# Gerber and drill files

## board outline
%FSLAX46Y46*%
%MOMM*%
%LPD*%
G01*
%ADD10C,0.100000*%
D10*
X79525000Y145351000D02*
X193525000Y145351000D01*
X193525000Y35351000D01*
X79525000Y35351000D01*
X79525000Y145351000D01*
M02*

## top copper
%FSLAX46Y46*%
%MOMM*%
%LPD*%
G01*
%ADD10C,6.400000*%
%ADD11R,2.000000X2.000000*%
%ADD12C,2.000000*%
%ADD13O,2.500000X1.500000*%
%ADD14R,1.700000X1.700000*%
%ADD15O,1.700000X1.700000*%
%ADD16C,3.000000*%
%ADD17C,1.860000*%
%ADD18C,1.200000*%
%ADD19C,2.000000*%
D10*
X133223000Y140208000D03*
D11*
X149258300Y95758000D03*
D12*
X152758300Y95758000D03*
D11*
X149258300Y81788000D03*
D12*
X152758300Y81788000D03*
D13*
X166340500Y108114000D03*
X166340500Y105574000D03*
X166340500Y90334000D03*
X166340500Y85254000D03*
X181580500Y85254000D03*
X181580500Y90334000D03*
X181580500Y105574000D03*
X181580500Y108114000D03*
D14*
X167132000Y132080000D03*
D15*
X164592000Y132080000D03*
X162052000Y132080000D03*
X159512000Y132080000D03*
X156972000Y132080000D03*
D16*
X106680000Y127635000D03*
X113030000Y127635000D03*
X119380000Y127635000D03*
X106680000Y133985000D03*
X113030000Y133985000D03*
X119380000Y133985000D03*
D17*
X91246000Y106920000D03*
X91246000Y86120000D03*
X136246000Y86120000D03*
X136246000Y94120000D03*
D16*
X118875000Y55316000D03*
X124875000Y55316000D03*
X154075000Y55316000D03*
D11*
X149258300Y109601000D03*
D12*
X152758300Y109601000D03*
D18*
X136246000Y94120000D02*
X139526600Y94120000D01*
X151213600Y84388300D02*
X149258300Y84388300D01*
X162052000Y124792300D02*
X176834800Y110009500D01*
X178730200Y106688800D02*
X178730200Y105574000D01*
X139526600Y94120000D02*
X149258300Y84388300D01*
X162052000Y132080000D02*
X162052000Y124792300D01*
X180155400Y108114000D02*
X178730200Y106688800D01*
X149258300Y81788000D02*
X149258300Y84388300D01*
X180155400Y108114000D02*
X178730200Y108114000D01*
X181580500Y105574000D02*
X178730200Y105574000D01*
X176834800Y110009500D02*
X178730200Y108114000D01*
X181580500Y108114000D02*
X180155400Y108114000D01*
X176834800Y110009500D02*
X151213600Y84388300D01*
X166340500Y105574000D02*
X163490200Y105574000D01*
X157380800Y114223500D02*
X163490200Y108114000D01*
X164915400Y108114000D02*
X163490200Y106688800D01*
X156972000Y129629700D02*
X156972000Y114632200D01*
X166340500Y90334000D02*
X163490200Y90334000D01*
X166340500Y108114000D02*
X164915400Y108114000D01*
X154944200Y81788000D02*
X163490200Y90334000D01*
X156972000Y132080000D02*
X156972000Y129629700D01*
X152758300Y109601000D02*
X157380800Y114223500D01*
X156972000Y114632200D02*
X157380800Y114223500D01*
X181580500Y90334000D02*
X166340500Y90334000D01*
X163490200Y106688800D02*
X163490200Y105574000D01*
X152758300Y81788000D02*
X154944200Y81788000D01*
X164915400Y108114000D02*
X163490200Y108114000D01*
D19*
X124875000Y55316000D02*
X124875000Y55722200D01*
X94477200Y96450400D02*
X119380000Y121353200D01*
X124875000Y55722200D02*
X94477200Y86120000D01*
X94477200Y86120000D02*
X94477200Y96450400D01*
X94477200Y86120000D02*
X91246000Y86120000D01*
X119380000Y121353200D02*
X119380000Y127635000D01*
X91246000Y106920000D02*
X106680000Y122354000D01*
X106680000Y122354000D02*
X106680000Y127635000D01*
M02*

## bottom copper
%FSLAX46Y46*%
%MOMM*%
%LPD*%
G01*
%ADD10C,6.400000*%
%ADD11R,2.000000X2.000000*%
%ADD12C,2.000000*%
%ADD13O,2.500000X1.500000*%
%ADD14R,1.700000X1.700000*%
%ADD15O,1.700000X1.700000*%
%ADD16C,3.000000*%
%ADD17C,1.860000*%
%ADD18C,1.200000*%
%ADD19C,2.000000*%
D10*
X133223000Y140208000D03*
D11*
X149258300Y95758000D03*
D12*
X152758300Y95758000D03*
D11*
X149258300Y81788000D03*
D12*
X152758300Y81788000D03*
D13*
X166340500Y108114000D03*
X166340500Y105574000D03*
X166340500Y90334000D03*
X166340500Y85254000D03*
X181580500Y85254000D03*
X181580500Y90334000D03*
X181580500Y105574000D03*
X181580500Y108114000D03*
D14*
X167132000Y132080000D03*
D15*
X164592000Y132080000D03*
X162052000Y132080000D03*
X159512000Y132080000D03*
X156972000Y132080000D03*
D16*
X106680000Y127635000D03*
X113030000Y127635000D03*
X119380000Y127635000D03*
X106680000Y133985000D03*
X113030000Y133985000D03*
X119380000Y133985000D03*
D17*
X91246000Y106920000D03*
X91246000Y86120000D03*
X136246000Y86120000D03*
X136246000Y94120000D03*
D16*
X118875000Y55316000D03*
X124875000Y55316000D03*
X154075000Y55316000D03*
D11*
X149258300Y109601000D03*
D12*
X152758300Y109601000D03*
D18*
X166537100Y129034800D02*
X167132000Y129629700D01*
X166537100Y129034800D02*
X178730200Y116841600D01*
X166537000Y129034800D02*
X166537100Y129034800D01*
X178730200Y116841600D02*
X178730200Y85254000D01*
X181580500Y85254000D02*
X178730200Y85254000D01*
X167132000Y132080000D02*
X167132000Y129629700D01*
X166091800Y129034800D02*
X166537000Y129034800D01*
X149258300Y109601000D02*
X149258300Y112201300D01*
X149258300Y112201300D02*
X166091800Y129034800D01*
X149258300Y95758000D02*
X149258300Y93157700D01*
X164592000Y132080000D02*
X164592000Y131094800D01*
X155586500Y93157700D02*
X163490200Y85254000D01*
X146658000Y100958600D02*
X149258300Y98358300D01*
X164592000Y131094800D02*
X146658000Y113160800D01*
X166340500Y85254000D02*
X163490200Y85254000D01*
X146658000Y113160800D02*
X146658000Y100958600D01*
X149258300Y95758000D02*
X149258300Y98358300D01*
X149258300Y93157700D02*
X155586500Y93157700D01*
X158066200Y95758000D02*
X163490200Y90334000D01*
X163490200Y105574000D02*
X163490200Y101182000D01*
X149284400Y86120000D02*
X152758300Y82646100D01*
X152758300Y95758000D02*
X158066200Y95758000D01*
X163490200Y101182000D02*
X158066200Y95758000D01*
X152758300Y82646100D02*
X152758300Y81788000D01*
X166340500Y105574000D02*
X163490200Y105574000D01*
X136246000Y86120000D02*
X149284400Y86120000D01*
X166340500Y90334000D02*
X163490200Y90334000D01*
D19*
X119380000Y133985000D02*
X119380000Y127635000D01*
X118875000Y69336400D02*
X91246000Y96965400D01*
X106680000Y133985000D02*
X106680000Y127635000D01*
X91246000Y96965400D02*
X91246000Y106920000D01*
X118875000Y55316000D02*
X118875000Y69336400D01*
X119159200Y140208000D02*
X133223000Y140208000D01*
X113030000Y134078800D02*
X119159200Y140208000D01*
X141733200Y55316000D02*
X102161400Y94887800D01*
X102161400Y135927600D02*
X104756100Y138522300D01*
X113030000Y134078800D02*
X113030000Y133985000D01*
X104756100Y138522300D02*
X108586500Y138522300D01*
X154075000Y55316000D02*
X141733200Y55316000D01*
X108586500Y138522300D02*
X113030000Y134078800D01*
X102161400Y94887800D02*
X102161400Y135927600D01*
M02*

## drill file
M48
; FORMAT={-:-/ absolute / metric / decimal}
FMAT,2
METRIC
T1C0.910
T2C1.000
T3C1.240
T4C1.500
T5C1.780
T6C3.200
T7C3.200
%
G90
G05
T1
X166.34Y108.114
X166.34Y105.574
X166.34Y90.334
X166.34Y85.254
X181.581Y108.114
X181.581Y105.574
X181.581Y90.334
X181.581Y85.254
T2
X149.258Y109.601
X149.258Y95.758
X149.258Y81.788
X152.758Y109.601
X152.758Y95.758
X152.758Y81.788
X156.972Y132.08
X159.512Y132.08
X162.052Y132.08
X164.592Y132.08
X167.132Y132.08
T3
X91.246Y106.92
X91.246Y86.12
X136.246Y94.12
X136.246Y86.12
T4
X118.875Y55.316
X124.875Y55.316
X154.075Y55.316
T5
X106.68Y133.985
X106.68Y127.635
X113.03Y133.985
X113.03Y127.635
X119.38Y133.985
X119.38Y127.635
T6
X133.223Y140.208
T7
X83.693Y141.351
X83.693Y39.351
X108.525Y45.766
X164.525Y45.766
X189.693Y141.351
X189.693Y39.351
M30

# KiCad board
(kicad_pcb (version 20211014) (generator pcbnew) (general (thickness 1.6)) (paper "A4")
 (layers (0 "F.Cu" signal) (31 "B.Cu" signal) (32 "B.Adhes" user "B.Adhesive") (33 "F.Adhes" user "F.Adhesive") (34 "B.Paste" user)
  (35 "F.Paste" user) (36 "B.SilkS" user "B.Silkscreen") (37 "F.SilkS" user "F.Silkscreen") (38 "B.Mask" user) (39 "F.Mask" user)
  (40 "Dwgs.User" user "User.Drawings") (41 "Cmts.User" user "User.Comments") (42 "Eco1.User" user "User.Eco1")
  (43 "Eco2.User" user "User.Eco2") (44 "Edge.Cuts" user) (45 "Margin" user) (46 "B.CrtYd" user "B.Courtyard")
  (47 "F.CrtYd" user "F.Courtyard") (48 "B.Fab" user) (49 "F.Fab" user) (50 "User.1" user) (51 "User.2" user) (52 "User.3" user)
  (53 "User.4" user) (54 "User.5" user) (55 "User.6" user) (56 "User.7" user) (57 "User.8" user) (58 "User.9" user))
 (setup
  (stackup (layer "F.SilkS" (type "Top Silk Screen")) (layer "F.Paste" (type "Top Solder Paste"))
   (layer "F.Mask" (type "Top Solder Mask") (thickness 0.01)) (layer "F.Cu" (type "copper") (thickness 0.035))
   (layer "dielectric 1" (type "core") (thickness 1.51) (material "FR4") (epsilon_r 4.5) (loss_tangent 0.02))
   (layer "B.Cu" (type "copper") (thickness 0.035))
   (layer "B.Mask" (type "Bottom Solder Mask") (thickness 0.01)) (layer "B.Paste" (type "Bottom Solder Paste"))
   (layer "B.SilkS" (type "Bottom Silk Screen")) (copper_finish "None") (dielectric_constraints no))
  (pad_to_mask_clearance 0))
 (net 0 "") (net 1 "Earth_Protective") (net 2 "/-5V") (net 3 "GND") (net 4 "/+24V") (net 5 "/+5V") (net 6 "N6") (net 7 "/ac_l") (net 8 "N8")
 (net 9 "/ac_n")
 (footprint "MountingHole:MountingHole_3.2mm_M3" (layer "F.Cu") (at 189.693 -141.351)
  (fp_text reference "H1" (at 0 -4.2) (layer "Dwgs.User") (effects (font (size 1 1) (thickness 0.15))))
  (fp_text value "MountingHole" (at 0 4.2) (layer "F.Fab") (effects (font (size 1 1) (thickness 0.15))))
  (pad "" np_thru_hole circle (at 0 0) (size 3.2 3.2) (drill 3.2) (layers *.Cu *.Mask)))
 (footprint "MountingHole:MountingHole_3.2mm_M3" (layer "F.Cu") (at 83.693 -39.351)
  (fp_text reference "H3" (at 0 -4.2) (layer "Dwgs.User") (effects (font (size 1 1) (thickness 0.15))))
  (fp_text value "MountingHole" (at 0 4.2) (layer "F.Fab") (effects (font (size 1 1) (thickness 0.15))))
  (pad "" np_thru_hole circle (at 0 0) (size 3.2 3.2) (drill 3.2) (layers *.Cu *.Mask)))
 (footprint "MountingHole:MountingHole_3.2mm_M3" (layer "F.Cu") (at 83.693 -141.351)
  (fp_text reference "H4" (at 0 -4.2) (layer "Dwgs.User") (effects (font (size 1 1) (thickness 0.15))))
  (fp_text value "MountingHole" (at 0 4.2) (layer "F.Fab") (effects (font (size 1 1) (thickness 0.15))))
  (pad "" np_thru_hole circle (at 0 0) (size 3.2 3.2) (drill 3.2) (layers *.Cu *.Mask)))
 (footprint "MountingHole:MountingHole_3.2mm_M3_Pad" (layer "F.Cu") (at 133.223 -140.208)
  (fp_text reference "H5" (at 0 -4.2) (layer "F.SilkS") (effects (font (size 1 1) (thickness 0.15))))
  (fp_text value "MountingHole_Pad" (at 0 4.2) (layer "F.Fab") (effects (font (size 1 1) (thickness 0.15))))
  (pad "1" thru_hole circle (at 0 0) (size 6.4 6.4) (drill 3.2) (layers *.Cu *.Mask) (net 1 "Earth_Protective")))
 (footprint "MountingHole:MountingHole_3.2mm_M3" (layer "F.Cu") (at 189.693 -39.351)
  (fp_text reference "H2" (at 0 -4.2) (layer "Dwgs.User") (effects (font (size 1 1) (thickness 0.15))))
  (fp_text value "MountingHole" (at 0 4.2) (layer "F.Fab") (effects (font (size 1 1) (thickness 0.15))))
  (pad "" np_thru_hole circle (at 0 0) (size 3.2 3.2) (drill 3.2) (layers *.Cu *.Mask)))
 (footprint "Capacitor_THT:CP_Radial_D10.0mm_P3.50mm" (layer "F.Cu") (at 149.2583 -95.758)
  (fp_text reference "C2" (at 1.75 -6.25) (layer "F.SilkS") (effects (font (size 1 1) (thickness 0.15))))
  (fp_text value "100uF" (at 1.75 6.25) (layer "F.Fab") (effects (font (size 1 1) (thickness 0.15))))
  (pad "1" thru_hole rect (at 0 0) (size 2 2) (drill 1) (layers *.Cu *.Mask) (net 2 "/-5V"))
  (pad "2" thru_hole circle (at 3.5 0) (size 2 2) (drill 1) (layers *.Cu *.Mask) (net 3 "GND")))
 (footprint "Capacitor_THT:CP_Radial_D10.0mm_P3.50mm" (layer "F.Cu") (at 149.2583 -81.788)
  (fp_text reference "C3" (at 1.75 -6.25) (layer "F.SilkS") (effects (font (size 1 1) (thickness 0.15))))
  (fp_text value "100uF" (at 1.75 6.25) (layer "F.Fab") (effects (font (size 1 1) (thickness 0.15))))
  (pad "1" thru_hole rect (at 0 0) (size 2 2) (drill 1) (layers *.Cu *.Mask) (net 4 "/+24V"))
  (pad "2" thru_hole circle (at 3.5 0) (size 2 2) (drill 1) (layers *.Cu *.Mask) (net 3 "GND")))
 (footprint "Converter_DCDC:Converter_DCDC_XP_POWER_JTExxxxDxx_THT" (layer "F.Cu") (at 166.3405 -108.114)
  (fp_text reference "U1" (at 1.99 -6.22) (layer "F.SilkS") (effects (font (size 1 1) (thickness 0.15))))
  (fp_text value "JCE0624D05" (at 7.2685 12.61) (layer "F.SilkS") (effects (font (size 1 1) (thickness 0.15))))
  (pad "2" thru_hole oval (at 0 0) (size 2.5 1.5) (drill 0.91) (layers *.Cu *.Mask) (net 3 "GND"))
  (pad "3" thru_hole oval (at 0 2.54) (size 2.5 1.5) (drill 0.91) (layers *.Cu *.Mask) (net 3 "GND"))
  (pad "9" thru_hole oval (at 0 17.78) (size 2.5 1.5) (drill 0.91) (layers *.Cu *.Mask) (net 3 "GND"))
  (pad "11" thru_hole oval (at 0 22.86) (size 2.5 1.5) (drill 0.91) (layers *.Cu *.Mask) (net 2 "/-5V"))
  (pad "14" thru_hole oval (at 15.24 22.86) (size 2.5 1.5) (drill 0.91) (layers *.Cu *.Mask) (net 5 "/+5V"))
  (pad "16" thru_hole oval (at 15.24 17.78) (size 2.5 1.5) (drill 0.91) (layers *.Cu *.Mask) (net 3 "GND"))
  (pad "22" thru_hole oval (at 15.24 2.54) (size 2.5 1.5) (drill 0.91) (layers *.Cu *.Mask) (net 4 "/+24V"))
  (pad "23" thru_hole oval (at 15.24 0) (size 2.5 1.5) (drill 0.91) (layers *.Cu *.Mask) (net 4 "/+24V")))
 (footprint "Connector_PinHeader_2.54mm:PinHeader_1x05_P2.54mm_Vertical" (layer "F.Cu") (at 167.132 -132.08 -90)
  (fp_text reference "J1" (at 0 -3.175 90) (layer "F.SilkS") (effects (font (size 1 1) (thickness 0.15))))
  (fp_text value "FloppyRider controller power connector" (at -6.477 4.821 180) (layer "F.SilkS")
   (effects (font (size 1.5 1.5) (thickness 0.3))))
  (pad "1" thru_hole rect (at 0 0 270) (size 1.7 1.7) (drill 1) (layers *.Cu *.Mask) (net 5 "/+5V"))
  (pad "2" thru_hole oval (at 0 2.54 270) (size 1.7 1.7) (drill 1) (layers *.Cu *.Mask) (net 2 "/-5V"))
  (pad "3" thru_hole oval (at 0 5.08 270) (size 1.7 1.7) (drill 1) (layers *.Cu *.Mask) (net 4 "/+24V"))
  (pad "4" thru_hole oval (at 0 7.62 270) (size 1.7 1.7) (drill 1) (layers *.Cu *.Mask) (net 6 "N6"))
  (pad "5" thru_hole oval (at 0 10.16 270) (size 1.7 1.7) (drill 1) (layers *.Cu *.Mask) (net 3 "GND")))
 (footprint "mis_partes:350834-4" (layer "F.Cu") (at 102.87 -123.825)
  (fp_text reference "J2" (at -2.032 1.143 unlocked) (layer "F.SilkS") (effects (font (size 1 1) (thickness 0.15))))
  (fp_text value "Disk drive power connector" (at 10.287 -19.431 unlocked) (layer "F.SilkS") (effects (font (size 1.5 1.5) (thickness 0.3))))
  (pad "1" thru_hole circle (at 3.81 -3.81) (size 3 3) (drill 1.78) (layers *.Cu *.Mask) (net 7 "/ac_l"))
  (pad "2" thru_hole circle (at 10.16 -3.81) (size 3 3) (drill 1.78) (layers *.Cu *.Mask) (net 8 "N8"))
  (pad "3" thru_hole circle (at 16.51 -3.81) (size 3 3) (drill 1.78) (layers *.Cu *.Mask) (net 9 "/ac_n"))
  (pad "4" thru_hole circle (at 3.81 -10.16) (size 3 3) (drill 1.78) (layers *.Cu *.Mask) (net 7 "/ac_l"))
  (pad "5" thru_hole circle (at 10.16 -10.16) (size 3 3) (drill 1.78) (layers *.Cu *.Mask) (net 1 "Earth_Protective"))
  (pad "6" thru_hole circle (at 16.51 -10.16) (size 3 3) (drill 1.78) (layers *.Cu *.Mask) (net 9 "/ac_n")))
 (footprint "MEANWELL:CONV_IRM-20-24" (layer "F.Cu") (at 114.046 -96.52)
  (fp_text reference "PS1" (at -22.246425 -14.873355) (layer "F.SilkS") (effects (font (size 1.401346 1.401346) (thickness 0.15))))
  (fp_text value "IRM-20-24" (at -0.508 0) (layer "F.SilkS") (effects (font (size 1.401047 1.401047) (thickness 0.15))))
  (pad "1" thru_hole circle locked (at -22.8 -10.4) (size 1.86 1.86) (drill 1.24) (layers *.Cu *.Mask) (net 7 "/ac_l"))
  (pad "2" thru_hole circle locked (at -22.8 10.4) (size 1.86 1.86) (drill 1.24) (layers *.Cu *.Mask) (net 9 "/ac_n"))
  (pad "3" thru_hole circle locked (at 22.2 10.4) (size 1.86 1.86) (drill 1.24) (layers *.Cu *.Mask) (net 3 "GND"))
  (pad "4" thru_hole circle locked (at 22.2 2.4) (size 1.86 1.86) (drill 1.24) (layers *.Cu *.Mask) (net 4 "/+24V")))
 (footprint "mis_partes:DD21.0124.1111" (layer "F.Cu") (at 104.025 -36.266)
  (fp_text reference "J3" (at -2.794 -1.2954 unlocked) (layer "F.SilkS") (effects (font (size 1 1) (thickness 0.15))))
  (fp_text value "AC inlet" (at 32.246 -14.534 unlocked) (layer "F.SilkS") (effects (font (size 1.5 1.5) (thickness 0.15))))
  (pad "" np_thru_hole circle (at 4.5 -9.5) (size 3.2 3.2) (drill 3.2) (layers F&B.Cu *.Mask))
  (pad "" np_thru_hole circle (at 60.5 -9.5) (size 3.2 3.2) (drill 3.2) (layers F&B.Cu *.Mask))
  (pad "1" thru_hole circle (at 14.85 -19.05) (size 3 3) (drill 1.5) (layers *.Cu *.Mask) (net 7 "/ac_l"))
  (pad "2" thru_hole circle (at 20.85 -19.05) (size 3 3) (drill 1.5) (layers *.Cu *.Mask) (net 9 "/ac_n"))
  (pad "3" thru_hole circle (at 50.05 -19.05) (size 3 3) (drill 1.5) (layers *.Cu *.Mask) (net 1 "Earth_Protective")))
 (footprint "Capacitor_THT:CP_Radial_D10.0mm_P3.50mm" (layer "F.Cu") (at 149.2583 -109.601)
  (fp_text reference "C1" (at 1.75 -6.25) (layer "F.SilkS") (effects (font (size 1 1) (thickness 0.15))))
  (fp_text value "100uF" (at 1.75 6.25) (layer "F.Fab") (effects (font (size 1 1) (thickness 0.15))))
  (pad "1" thru_hole rect (at 0 0) (size 2 2) (drill 1) (layers *.Cu *.Mask) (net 5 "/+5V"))
  (pad "2" thru_hole circle (at 3.5 0) (size 2 2) (drill 1) (layers *.Cu *.Mask) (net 3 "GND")))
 (gr_rect (start 79.525 -145.351) (end 193.525 -35.351) (layer "Edge.Cuts") (width 0.1) (fill none))
 (segment (start 166.5371 -129.0348) (end 167.132 -129.6297) (width 1.2) (layer "B.Cu") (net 5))
 (segment (start 166.5371 -129.0348) (end 178.7302 -116.8416) (width 1.2) (layer "B.Cu") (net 5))
 (segment (start 166.537 -129.0348) (end 166.5371 -129.0348) (width 1.2) (layer "B.Cu") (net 5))
 (segment (start 178.7302 -116.8416) (end 178.7302 -85.254) (width 1.2) (layer "B.Cu") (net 5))
 (segment (start 181.5805 -85.254) (end 178.7302 -85.254) (width 1.2) (layer "B.Cu") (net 5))
 (segment (start 167.132 -132.08) (end 167.132 -129.6297) (width 1.2) (layer "B.Cu") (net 5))
 (segment (start 166.0918 -129.0348) (end 166.537 -129.0348) (width 1.2) (layer "B.Cu") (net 5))
 (segment (start 149.2583 -109.601) (end 149.2583 -112.2013) (width 1.2) (layer "B.Cu") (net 5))
 (segment (start 149.2583 -112.2013) (end 166.0918 -129.0348) (width 1.2) (layer "B.Cu") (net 5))
 (segment (start 149.2583 -95.758) (end 149.2583 -93.1577) (width 1.2) (layer "B.Cu") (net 2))
 (segment (start 164.592 -132.08) (end 164.592 -131.0948) (width 1.2) (layer "B.Cu") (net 2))
 (segment (start 155.5865 -93.1577) (end 163.4902 -85.254) (width 1.2) (layer "B.Cu") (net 2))
 (segment (start 146.658 -100.9586) (end 149.2583 -98.3583) (width 1.2) (layer "B.Cu") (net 2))
 (segment (start 164.592 -131.0948) (end 146.658 -113.1608) (width 1.2) (layer "B.Cu") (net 2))
 (segment (start 166.3405 -85.254) (end 163.4902 -85.254) (width 1.2) (layer "B.Cu") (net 2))
 (segment (start 146.658 -113.1608) (end 146.658 -100.9586) (width 1.2) (layer "B.Cu") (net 2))
 (segment (start 149.2583 -95.758) (end 149.2583 -98.3583) (width 1.2) (layer "B.Cu") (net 2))
 (segment (start 149.2583 -93.1577) (end 155.5865 -93.1577) (width 1.2) (layer "B.Cu") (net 2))
 (segment (start 136.246 -94.12) (end 139.5266 -94.12) (width 1.2) (layer "F.Cu") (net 4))
 (segment (start 151.2136 -84.3883) (end 149.2583 -84.3883) (width 1.2) (layer "F.Cu") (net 4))
 (segment (start 162.052 -124.7923) (end 176.8348 -110.0095) (width 1.2) (layer "F.Cu") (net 4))
 (segment (start 178.7302 -106.6888) (end 178.7302 -105.574) (width 1.2) (layer "F.Cu") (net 4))
 (segment (start 139.5266 -94.12) (end 149.2583 -84.3883) (width 1.2) (layer "F.Cu") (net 4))
 (segment (start 162.052 -132.08) (end 162.052 -124.7923) (width 1.2) (layer "F.Cu") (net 4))
 (segment (start 180.1554 -108.114) (end 178.7302 -106.6888) (width 1.2) (layer "F.Cu") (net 4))
 (segment (start 149.2583 -81.788) (end 149.2583 -84.3883) (width 1.2) (layer "F.Cu") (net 4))
 (segment (start 180.1554 -108.114) (end 178.7302 -108.114) (width 1.2) (layer "F.Cu") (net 4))
 (segment (start 181.5805 -105.574) (end 178.7302 -105.574) (width 1.2) (layer "F.Cu") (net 4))
 (segment (start 176.8348 -110.0095) (end 178.7302 -108.114) (width 1.2) (layer "F.Cu") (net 4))
 (segment (start 181.5805 -108.114) (end 180.1554 -108.114) (width 1.2) (layer "F.Cu") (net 4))
 (segment (start 176.8348 -110.0095) (end 151.2136 -84.3883) (width 1.2) (layer "F.Cu") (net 4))
 (segment (start 166.3405 -105.574) (end 163.4902 -105.574) (width 1.2) (layer "F.Cu") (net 3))
 (segment (start 157.3808 -114.2235) (end 163.4902 -108.114) (width 1.2) (layer "F.Cu") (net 3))
 (segment (start 164.9154 -108.114) (end 163.4902 -106.6888) (width 1.2) (layer "F.Cu") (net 3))
 (segment (start 156.972 -129.6297) (end 156.972 -114.6322) (width 1.2) (layer "F.Cu") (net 3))
 (segment (start 166.3405 -90.334) (end 163.4902 -90.334) (width 1.2) (layer "F.Cu") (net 3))
 (segment (start 166.3405 -108.114) (end 164.9154 -108.114) (width 1.2) (layer "F.Cu") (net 3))
 (segment (start 154.9442 -81.788) (end 163.4902 -90.334) (width 1.2) (layer "F.Cu") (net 3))
 (segment (start 156.972 -132.08) (end 156.972 -129.6297) (width 1.2) (layer "F.Cu") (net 3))
 (segment (start 152.7583 -109.601) (end 157.3808 -114.2235) (width 1.2) (layer "F.Cu") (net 3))
 (segment (start 156.972 -114.6322) (end 157.3808 -114.2235) (width 1.2) (layer "F.Cu") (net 3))
 (segment (start 181.5805 -90.334) (end 166.3405 -90.334) (width 1.2) (layer "F.Cu") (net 3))
 (segment (start 163.4902 -106.6888) (end 163.4902 -105.574) (width 1.2) (layer "F.Cu") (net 3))
 (segment (start 152.7583 -81.788) (end 154.9442 -81.788) (width 1.2) (layer "F.Cu") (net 3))
 (segment (start 164.9154 -108.114) (end 163.4902 -108.114) (width 1.2) (layer "F.Cu") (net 3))
 (segment (start 158.0662 -95.758) (end 163.4902 -90.334) (width 1.2) (layer "B.Cu") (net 3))
 (segment (start 163.4902 -105.574) (end 163.4902 -101.182) (width 1.2) (layer "B.Cu") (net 3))
 (segment (start 149.2844 -86.12) (end 152.7583 -82.6461) (width 1.2) (layer "B.Cu") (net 3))
 (segment (start 152.7583 -95.758) (end 158.0662 -95.758) (width 1.2) (layer "B.Cu") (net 3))
 (segment (start 163.4902 -101.182) (end 158.0662 -95.758) (width 1.2) (layer "B.Cu") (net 3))
 (segment (start 152.7583 -82.6461) (end 152.7583 -81.788) (width 1.2) (layer "B.Cu") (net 3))
 (segment (start 166.3405 -105.574) (end 163.4902 -105.574) (width 1.2) (layer "B.Cu") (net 3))
 (segment (start 136.246 -86.12) (end 149.2844 -86.12) (width 1.2) (layer "B.Cu") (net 3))
 (segment (start 166.3405 -90.334) (end 163.4902 -90.334) (width 1.2) (layer "B.Cu") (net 3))
 (segment (start 124.875 -55.316) (end 124.875 -55.7222) (width 2) (layer "F.Cu") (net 9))
 (segment (start 94.4772 -96.4504) (end 119.38 -121.3532) (width 2) (layer "F.Cu") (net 9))
 (segment (start 124.875 -55.7222) (end 94.4772 -86.12) (width 2) (layer "F.Cu") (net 9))
 (segment (start 94.4772 -86.12) (end 94.4772 -96.4504) (width 2) (layer "F.Cu") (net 9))
 (segment (start 94.4772 -86.12) (end 91.246 -86.12) (width 2) (layer "F.Cu") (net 9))
 (segment (start 119.38 -121.3532) (end 119.38 -127.635) (width 2) (layer "F.Cu") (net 9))
 (segment (start 119.38 -133.985) (end 119.38 -127.635) (width 2) (layer "B.Cu") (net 9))
 (segment (start 91.246 -106.92) (end 106.68 -122.354) (width 2) (layer "F.Cu") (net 7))
 (segment (start 106.68 -122.354) (end 106.68 -127.635) (width 2) (layer "F.Cu") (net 7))
 (segment (start 118.875 -69.3364) (end 91.246 -96.9654) (width 2) (layer "B.Cu") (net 7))
 (segment (start 106.68 -133.985) (end 106.68 -127.635) (width 2) (layer "B.Cu") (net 7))
 (segment (start 91.246 -96.9654) (end 91.246 -106.92) (width 2) (layer "B.Cu") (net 7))
 (segment (start 118.875 -55.316) (end 118.875 -69.3364) (width 2) (layer "B.Cu") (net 7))
 (segment (start 119.1592 -140.208) (end 133.223 -140.208) (width 2) (layer "B.Cu") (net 1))
 (segment (start 113.03 -134.0788) (end 119.1592 -140.208) (width 2) (layer "B.Cu") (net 1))
 (segment (start 141.7332 -55.316) (end 102.1614 -94.8878) (width 2) (layer "B.Cu") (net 1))
 (segment (start 102.1614 -135.9276) (end 104.7561 -138.5223) (width 2) (layer "B.Cu") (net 1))
 (segment (start 113.03 -134.0788) (end 113.03 -133.985) (width 2) (layer "B.Cu") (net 1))
 (segment (start 104.7561 -138.5223) (end 108.5865 -138.5223) (width 2) (layer "B.Cu") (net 1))
 (segment (start 154.075 -55.316) (end 141.7332 -55.316) (width 2) (layer "B.Cu") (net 1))
 (segment (start 108.5865 -138.5223) (end 113.03 -134.0788) (width 2) (layer "B.Cu") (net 1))
 (segment (start 102.1614 -94.8878) (end 102.1614 -135.9276) (width 2) (layer "B.Cu") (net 1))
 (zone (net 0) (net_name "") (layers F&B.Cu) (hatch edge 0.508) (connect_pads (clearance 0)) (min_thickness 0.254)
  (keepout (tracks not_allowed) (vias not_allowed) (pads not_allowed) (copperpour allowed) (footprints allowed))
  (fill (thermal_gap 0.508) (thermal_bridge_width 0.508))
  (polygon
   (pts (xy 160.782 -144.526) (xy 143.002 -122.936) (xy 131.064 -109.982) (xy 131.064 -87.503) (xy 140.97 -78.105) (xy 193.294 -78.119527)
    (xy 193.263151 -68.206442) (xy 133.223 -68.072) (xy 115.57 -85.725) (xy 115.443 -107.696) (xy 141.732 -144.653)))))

